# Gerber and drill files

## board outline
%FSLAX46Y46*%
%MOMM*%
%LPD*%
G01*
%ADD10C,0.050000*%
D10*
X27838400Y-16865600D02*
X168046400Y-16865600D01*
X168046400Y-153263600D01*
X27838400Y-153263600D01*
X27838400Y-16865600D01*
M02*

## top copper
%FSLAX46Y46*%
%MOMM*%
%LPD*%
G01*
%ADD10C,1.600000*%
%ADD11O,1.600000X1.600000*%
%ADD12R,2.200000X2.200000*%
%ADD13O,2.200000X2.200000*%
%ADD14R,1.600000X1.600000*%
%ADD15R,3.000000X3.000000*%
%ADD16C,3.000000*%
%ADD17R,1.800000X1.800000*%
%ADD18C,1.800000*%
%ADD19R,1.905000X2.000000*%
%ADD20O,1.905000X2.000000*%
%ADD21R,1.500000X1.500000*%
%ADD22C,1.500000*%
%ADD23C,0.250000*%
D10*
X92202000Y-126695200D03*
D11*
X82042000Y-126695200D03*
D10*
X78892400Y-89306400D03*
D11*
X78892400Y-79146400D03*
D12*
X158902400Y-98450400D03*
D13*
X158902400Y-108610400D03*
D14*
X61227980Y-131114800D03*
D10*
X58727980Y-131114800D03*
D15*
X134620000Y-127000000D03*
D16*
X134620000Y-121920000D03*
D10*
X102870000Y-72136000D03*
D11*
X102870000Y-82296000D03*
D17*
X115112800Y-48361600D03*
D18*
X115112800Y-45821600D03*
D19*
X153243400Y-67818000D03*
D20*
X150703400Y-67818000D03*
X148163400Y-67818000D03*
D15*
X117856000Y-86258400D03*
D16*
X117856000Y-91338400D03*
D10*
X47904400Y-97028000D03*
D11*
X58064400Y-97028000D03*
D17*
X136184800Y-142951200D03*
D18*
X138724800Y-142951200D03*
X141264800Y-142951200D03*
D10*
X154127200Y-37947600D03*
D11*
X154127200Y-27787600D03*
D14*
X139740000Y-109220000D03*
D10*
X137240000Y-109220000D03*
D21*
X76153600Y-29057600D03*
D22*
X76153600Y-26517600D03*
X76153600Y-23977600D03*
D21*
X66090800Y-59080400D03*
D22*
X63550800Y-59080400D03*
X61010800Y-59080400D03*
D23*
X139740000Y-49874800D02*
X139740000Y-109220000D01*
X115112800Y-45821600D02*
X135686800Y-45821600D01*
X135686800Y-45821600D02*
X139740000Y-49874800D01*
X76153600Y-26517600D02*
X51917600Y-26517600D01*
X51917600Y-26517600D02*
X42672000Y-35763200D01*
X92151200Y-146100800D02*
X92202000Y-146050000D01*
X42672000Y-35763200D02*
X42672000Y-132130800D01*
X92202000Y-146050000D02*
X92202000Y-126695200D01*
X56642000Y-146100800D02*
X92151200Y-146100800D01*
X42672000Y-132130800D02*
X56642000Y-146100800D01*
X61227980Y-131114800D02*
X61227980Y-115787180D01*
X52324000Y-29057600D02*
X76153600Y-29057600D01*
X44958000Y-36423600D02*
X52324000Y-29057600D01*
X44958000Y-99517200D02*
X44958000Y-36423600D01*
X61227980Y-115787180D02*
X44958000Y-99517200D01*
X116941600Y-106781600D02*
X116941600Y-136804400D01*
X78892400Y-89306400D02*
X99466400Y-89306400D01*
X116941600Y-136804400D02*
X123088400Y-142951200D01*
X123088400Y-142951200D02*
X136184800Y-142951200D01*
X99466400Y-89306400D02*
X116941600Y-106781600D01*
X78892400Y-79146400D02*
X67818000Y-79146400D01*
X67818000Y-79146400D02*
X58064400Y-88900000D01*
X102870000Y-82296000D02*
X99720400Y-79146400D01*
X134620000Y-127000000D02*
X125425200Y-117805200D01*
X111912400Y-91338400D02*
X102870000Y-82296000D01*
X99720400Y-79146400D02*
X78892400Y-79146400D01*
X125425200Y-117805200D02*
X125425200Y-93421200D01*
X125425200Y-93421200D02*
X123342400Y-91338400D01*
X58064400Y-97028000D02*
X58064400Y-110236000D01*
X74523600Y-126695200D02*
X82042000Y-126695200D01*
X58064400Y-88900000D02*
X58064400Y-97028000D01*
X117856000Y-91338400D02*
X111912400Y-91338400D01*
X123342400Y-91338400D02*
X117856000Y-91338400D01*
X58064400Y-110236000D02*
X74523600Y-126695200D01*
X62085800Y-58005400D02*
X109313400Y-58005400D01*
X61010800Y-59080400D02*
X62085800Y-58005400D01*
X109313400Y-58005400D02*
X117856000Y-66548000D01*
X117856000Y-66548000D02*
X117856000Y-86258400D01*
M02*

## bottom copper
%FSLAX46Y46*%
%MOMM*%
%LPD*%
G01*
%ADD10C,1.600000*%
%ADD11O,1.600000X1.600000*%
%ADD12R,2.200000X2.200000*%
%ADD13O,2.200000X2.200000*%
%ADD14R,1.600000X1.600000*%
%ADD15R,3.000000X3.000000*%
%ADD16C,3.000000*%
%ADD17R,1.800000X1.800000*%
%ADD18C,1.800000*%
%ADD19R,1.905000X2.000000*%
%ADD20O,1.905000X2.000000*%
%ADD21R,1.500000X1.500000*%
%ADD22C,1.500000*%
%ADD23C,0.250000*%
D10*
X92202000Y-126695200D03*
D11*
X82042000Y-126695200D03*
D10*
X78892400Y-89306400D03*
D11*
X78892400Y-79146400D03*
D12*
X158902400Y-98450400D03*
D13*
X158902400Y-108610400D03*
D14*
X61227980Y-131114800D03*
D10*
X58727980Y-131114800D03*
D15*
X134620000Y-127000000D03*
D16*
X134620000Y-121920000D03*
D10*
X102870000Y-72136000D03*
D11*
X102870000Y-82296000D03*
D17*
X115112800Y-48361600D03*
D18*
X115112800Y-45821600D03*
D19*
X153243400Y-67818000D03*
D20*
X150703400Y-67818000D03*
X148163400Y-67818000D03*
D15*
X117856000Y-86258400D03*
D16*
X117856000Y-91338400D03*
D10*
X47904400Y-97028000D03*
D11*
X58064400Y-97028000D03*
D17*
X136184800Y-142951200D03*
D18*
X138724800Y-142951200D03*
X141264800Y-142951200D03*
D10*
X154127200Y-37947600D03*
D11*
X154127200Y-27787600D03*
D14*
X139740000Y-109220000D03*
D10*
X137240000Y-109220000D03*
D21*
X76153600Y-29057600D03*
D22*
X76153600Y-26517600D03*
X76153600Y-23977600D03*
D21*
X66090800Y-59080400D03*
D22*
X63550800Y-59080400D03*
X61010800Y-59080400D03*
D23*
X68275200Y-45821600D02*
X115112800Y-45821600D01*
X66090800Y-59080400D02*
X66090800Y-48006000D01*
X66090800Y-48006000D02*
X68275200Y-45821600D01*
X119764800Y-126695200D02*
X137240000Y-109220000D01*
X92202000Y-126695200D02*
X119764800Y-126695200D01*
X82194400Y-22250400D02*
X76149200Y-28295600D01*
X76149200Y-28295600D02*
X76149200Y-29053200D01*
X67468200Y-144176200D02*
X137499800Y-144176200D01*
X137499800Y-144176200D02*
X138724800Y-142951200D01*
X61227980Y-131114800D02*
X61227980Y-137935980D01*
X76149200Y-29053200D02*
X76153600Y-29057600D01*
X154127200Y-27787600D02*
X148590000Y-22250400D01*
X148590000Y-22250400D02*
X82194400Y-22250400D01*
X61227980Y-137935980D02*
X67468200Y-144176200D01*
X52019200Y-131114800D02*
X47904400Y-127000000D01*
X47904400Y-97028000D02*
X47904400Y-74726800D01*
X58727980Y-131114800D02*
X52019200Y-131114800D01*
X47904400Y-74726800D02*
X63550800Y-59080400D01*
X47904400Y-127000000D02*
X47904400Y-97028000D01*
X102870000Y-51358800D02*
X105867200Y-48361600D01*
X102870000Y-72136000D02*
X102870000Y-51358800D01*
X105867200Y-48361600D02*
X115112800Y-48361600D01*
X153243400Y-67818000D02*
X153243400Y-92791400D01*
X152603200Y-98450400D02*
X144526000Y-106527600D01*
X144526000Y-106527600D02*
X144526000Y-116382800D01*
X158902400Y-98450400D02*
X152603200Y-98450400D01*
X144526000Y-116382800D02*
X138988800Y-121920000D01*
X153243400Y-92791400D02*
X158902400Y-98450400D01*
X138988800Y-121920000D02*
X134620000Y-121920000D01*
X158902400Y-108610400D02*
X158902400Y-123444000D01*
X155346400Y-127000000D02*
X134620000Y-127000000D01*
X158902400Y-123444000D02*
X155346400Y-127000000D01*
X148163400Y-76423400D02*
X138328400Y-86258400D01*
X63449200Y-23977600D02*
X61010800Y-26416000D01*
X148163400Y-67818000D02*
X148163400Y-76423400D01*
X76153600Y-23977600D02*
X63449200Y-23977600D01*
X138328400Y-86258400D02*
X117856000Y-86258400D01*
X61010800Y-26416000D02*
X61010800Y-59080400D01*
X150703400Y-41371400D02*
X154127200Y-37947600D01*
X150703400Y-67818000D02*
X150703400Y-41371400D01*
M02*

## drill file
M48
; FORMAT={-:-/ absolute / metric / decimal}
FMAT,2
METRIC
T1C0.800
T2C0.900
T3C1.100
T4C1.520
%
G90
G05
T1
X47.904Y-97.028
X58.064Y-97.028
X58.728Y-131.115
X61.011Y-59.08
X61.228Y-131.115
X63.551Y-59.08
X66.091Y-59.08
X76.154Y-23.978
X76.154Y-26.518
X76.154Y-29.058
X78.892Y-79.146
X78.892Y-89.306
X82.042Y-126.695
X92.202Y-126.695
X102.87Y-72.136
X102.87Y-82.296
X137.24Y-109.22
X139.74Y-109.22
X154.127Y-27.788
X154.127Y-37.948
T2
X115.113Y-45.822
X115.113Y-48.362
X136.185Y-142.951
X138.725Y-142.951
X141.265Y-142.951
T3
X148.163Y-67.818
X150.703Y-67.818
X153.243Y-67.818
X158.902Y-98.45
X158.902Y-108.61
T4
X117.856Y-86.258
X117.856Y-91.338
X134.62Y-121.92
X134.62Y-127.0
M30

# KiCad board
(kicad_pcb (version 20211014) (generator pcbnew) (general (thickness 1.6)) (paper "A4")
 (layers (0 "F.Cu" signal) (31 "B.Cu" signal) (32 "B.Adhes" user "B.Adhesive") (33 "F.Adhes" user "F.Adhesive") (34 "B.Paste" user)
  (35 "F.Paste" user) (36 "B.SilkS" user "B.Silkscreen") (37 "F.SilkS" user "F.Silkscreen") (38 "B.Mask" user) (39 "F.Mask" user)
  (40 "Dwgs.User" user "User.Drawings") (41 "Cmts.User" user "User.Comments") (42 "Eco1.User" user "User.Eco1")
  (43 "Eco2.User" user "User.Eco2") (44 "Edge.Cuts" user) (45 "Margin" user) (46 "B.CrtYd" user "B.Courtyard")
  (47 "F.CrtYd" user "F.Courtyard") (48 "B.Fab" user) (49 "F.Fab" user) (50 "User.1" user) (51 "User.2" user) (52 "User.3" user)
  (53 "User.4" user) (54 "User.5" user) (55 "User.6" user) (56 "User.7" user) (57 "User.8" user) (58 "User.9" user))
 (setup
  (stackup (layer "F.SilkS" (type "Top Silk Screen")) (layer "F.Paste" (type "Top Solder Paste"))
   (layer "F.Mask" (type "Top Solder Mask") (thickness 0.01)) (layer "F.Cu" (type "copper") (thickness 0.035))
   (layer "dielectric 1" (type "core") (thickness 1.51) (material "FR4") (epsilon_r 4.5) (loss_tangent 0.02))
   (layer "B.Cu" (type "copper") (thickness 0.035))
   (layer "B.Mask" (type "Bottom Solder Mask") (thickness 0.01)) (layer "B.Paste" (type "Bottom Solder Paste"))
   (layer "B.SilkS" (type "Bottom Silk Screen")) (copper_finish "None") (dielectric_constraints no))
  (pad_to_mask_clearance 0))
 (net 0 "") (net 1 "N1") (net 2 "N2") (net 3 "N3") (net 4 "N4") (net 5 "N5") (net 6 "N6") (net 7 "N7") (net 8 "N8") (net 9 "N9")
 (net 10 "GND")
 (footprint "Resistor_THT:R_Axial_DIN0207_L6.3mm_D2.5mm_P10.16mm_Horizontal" (layer "F.Cu") (at 92.202 126.6952 180)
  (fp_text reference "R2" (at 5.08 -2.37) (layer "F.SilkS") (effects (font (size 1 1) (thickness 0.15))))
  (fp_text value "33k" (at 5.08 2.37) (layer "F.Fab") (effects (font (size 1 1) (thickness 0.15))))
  (pad "1" thru_hole circle (at 0 0 180) (size 1.6 1.6) (drill 0.8) (layers *.Cu *.Mask) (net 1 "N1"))
  (pad "2" thru_hole oval (at 10.16 0 180) (size 1.6 1.6) (drill 0.8) (layers *.Cu *.Mask) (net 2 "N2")))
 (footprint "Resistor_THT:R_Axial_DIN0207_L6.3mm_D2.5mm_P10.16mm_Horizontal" (layer "F.Cu") (at 78.8924 89.3064 90)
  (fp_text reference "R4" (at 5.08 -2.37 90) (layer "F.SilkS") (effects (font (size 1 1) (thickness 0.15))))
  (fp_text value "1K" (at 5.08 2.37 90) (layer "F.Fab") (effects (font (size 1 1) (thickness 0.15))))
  (pad "1" thru_hole circle (at 0 0 90) (size 1.6 1.6) (drill 0.8) (layers *.Cu *.Mask) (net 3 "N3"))
  (pad "2" thru_hole oval (at 10.16 0 90) (size 1.6 1.6) (drill 0.8) (layers *.Cu *.Mask) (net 2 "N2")))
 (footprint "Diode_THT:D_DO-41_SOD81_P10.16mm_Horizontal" (layer "F.Cu") (at 158.9024 98.4504 -90)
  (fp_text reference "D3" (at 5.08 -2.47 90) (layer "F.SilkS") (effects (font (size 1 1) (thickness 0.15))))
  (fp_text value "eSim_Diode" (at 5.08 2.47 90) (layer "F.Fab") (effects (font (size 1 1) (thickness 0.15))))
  (pad "1" thru_hole rect (at 0 0 270) (size 2.2 2.2) (drill 1.1) (layers *.Cu *.Mask) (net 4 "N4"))
  (pad "2" thru_hole oval (at 10.16 0 270) (size 2.2 2.2) (drill 1.1) (layers *.Cu *.Mask) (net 2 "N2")))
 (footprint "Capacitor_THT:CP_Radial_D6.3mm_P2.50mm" (layer "F.Cu") (at 61.22798 131.1148 180)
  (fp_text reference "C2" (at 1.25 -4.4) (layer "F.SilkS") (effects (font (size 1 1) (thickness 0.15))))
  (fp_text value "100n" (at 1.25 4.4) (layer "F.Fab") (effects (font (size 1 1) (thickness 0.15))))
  (pad "1" thru_hole rect (at 0 0 180) (size 1.6 1.6) (drill 0.8) (layers *.Cu *.Mask) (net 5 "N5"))
  (pad "2" thru_hole circle (at 2.5 0 180) (size 1.6 1.6) (drill 0.8) (layers *.Cu *.Mask) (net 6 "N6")))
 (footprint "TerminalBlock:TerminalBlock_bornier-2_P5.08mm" (layer "F.Cu") (at 134.62 127 90)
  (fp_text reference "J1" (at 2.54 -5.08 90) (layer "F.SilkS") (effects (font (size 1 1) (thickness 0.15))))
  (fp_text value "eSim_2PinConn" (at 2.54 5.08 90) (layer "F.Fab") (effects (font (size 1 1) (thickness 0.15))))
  (pad "1" thru_hole rect (at 0 0 90) (size 3 3) (drill 1.52) (layers *.Cu *.Mask) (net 2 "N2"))
  (pad "2" thru_hole circle (at 5.08 0 90) (size 3 3) (drill 1.52) (layers *.Cu *.Mask) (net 4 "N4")))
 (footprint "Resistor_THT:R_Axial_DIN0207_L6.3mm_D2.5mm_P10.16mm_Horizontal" (layer "F.Cu") (at 102.87 72.136 -90)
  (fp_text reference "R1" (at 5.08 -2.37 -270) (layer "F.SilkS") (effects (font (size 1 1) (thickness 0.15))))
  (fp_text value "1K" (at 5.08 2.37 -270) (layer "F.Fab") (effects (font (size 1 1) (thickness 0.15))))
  (pad "1" thru_hole circle (at 0 0 270) (size 1.6 1.6) (drill 0.8) (layers *.Cu *.Mask) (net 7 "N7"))
  (pad "2" thru_hole oval (at 10.16 0 270) (size 1.6 1.6) (drill 0.8) (layers *.Cu *.Mask) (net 2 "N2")))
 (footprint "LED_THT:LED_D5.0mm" (layer "F.Cu") (at 115.1128 48.3616 90)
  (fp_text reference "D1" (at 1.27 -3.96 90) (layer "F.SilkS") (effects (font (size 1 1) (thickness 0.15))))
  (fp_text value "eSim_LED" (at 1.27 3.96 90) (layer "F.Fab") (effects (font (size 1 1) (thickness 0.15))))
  (pad "1" thru_hole rect (at 0 0 90) (size 1.8 1.8) (drill 0.9) (layers *.Cu *.Mask) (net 7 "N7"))
  (pad "2" thru_hole circle (at 2.54 0 90) (size 1.8 1.8) (drill 0.9) (layers *.Cu *.Mask) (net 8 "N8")))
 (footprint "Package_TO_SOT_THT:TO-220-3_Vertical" (layer "F.Cu") (at 153.2434 67.818 180)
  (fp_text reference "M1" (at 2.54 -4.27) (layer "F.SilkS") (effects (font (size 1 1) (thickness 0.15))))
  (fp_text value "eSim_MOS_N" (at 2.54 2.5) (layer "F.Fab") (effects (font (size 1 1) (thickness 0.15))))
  (pad "1" thru_hole rect (at 0 0 180) (size 1.905 2) (drill 1.1) (layers *.Cu *.Mask) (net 4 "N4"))
  (pad "2" thru_hole oval (at 2.54 0 180) (size 1.905 2) (drill 1.1) (layers *.Cu *.Mask) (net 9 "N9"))
  (pad "3" thru_hole oval (at 5.08 0 180) (size 1.905 2) (drill 1.1) (layers *.Cu *.Mask) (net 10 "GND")))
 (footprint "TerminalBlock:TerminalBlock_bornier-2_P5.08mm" (layer "F.Cu") (at 117.856 86.2584 -90)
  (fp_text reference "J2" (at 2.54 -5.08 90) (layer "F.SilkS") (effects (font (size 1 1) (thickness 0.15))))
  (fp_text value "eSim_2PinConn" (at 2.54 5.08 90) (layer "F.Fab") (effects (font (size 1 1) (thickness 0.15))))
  (pad "1" thru_hole rect (at 0 0 270) (size 3 3) (drill 1.52) (layers *.Cu *.Mask) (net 10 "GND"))
  (pad "2" thru_hole circle (at 5.08 0 270) (size 3 3) (drill 1.52) (layers *.Cu *.Mask) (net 2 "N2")))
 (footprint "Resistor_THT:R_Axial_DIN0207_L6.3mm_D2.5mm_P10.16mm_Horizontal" (layer "F.Cu") (at 47.9044 97.028)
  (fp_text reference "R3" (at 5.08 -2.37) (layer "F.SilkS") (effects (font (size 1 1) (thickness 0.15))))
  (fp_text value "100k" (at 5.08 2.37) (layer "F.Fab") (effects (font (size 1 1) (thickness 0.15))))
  (pad "1" thru_hole circle (at 0 0) (size 1.6 1.6) (drill 0.8) (layers *.Cu *.Mask) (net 6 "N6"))
  (pad "2" thru_hole oval (at 10.16 0) (size 1.6 1.6) (drill 0.8) (layers *.Cu *.Mask) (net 2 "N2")))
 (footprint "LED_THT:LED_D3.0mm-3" (layer "F.Cu") (at 136.1848 142.9512)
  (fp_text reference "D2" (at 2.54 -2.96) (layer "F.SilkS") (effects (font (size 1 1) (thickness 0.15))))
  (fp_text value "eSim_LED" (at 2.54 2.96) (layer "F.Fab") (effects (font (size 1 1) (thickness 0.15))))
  (pad "1" thru_hole rect (at 0 0) (size 1.8 1.8) (drill 0.9) (layers *.Cu *.Mask) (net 3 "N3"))
  (pad "2" thru_hole circle (at 2.54 0) (size 1.8 1.8) (drill 0.9) (layers *.Cu *.Mask) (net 5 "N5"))
  (pad "3" thru_hole circle (at 5.08 0) (size 1.8 1.8) (drill 0.9) (layers *.Cu *.Mask)))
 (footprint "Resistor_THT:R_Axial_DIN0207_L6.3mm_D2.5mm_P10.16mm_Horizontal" (layer "F.Cu") (at 154.1272 37.9476 90)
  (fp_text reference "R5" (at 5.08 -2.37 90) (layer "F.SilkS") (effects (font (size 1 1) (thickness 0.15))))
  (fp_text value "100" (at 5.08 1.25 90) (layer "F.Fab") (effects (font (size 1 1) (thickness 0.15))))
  (pad "1" thru_hole circle (at 0 0 90) (size 1.6 1.6) (drill 0.8) (layers *.Cu *.Mask) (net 9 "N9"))
  (pad "2" thru_hole oval (at 10.16 0 90) (size 1.6 1.6) (drill 0.8) (layers *.Cu *.Mask) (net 5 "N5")))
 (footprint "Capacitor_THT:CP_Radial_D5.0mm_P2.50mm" (layer "F.Cu") (at 139.74 109.22 180)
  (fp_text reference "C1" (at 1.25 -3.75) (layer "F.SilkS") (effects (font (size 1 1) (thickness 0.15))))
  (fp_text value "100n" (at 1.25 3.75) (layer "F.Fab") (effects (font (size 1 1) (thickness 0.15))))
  (pad "1" thru_hole rect (at 0 0 180) (size 1.6 1.6) (drill 0.8) (layers *.Cu *.Mask) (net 8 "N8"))
  (pad "2" thru_hole circle (at 2.5 0 180) (size 1.6 1.6) (drill 0.8) (layers *.Cu *.Mask) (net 1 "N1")))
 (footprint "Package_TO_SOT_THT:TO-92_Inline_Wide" (layer "F.Cu") (at 76.1536 29.0576 90)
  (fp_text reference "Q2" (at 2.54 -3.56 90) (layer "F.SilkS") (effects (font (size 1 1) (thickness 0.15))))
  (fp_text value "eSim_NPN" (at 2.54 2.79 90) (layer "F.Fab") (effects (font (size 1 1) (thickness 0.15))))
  (pad "1" thru_hole rect (at 0 0 90) (size 1.5 1.5) (drill 0.8) (layers *.Cu *.Mask) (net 5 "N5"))
  (pad "2" thru_hole circle (at 2.54 0 90) (size 1.5 1.5) (drill 0.8) (layers *.Cu *.Mask) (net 1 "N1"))
  (pad "3" thru_hole circle (at 5.08 0 90) (size 1.5 1.5) (drill 0.8) (layers *.Cu *.Mask) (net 10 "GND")))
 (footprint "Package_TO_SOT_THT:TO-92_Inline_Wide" (layer "F.Cu") (at 66.0908 59.0804 180)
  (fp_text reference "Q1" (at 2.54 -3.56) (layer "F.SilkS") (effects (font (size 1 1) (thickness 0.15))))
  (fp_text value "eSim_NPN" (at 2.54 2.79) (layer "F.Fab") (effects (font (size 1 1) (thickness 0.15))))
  (pad "1" thru_hole rect (at 0 0 180) (size 1.5 1.5) (drill 0.8) (layers *.Cu *.Mask) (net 8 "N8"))
  (pad "2" thru_hole circle (at 2.54 0 180) (size 1.5 1.5) (drill 0.8) (layers *.Cu *.Mask) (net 6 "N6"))
  (pad "3" thru_hole circle (at 5.08 0 180) (size 1.5 1.5) (drill 0.8) (layers *.Cu *.Mask) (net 10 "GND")))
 (gr_rect (start 27.8384 16.8656) (end 168.0464 153.2636) (layer "Edge.Cuts") (width 0.05) (fill none))
 (segment (start 139.74 49.8748) (end 139.74 109.22) (width 0.25) (layer "F.Cu") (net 8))
 (segment (start 115.1128 45.8216) (end 135.6868 45.8216) (width 0.25) (layer "F.Cu") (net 8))
 (segment (start 135.6868 45.8216) (end 139.74 49.8748) (width 0.25) (layer "F.Cu") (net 8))
 (segment (start 68.2752 45.8216) (end 115.1128 45.8216) (width 0.25) (layer "B.Cu") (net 8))
 (segment (start 66.0908 59.0804) (end 66.0908 48.006) (width 0.25) (layer "B.Cu") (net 8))
 (segment (start 66.0908 48.006) (end 68.2752 45.8216) (width 0.25) (layer "B.Cu") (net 8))
 (segment (start 76.1536 26.5176) (end 51.9176 26.5176) (width 0.25) (layer "F.Cu") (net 1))
 (segment (start 51.9176 26.5176) (end 42.672 35.7632) (width 0.25) (layer "F.Cu") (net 1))
 (segment (start 92.1512 146.1008) (end 92.202 146.05) (width 0.25) (layer "F.Cu") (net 1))
 (segment (start 42.672 35.7632) (end 42.672 132.1308) (width 0.25) (layer "F.Cu") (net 1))
 (segment (start 92.202 146.05) (end 92.202 126.6952) (width 0.25) (layer "F.Cu") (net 1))
 (segment (start 56.642 146.1008) (end 92.1512 146.1008) (width 0.25) (layer "F.Cu") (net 1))
 (segment (start 42.672 132.1308) (end 56.642 146.1008) (width 0.25) (layer "F.Cu") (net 1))
 (segment (start 119.7648 126.6952) (end 137.24 109.22) (width 0.25) (layer "B.Cu") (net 1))
 (segment (start 92.202 126.6952) (end 119.7648 126.6952) (width 0.25) (layer "B.Cu") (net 1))
 (segment (start 61.22798 131.1148) (end 61.22798 115.78718) (width 0.25) (layer "F.Cu") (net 5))
 (segment (start 52.324 29.0576) (end 76.1536 29.0576) (width 0.25) (layer "F.Cu") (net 5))
 (segment (start 44.958 36.4236) (end 52.324 29.0576) (width 0.25) (layer "F.Cu") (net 5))
 (segment (start 44.958 99.5172) (end 44.958 36.4236) (width 0.25) (layer "F.Cu") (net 5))
 (segment (start 61.22798 115.78718) (end 44.958 99.5172) (width 0.25) (layer "F.Cu") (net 5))
 (segment (start 82.1944 22.2504) (end 76.1492 28.2956) (width 0.25) (layer "B.Cu") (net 5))
 (segment (start 76.1492 28.2956) (end 76.1492 29.0532) (width 0.25) (layer "B.Cu") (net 5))
 (segment (start 67.4682 144.1762) (end 137.4998 144.1762) (width 0.25) (layer "B.Cu") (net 5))
 (segment (start 137.4998 144.1762) (end 138.7248 142.9512) (width 0.25) (layer "B.Cu") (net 5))
 (segment (start 61.22798 131.1148) (end 61.22798 137.93598) (width 0.25) (layer "B.Cu") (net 5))
 (segment (start 76.1492 29.0532) (end 76.1536 29.0576) (width 0.25) (layer "B.Cu") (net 5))
 (segment (start 154.1272 27.7876) (end 148.59 22.2504) (width 0.25) (layer "B.Cu") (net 5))
 (segment (start 148.59 22.2504) (end 82.1944 22.2504) (width 0.25) (layer "B.Cu") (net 5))
 (segment (start 61.22798 137.93598) (end 67.4682 144.1762) (width 0.25) (layer "B.Cu") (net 5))
 (segment (start 52.0192 131.1148) (end 47.9044 127) (width 0.25) (layer "B.Cu") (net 6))
 (segment (start 47.9044 97.028) (end 47.9044 74.7268) (width 0.25) (layer "B.Cu") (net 6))
 (segment (start 58.72798 131.1148) (end 52.0192 131.1148) (width 0.25) (layer "B.Cu") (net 6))
 (segment (start 47.9044 74.7268) (end 63.5508 59.0804) (width 0.25) (layer "B.Cu") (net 6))
 (segment (start 47.9044 127) (end 47.9044 97.028) (width 0.25) (layer "B.Cu") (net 6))
 (segment (start 102.87 51.3588) (end 105.8672 48.3616) (width 0.25) (layer "B.Cu") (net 7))
 (segment (start 102.87 72.136) (end 102.87 51.3588) (width 0.25) (layer "B.Cu") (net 7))
 (segment (start 105.8672 48.3616) (end 115.1128 48.3616) (width 0.25) (layer "B.Cu") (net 7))
 (segment (start 116.9416 106.7816) (end 116.9416 136.8044) (width 0.25) (layer "F.Cu") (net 3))
 (segment (start 78.8924 89.3064) (end 99.4664 89.3064) (width 0.25) (layer "F.Cu") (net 3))
 (segment (start 116.9416 136.8044) (end 123.0884 142.9512) (width 0.25) (layer "F.Cu") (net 3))
 (segment (start 123.0884 142.9512) (end 136.1848 142.9512) (width 0.25) (layer "F.Cu") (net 3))
 (segment (start 99.4664 89.3064) (end 116.9416 106.7816) (width 0.25) (layer "F.Cu") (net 3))
 (segment (start 153.2434 67.818) (end 153.2434 92.7914) (width 0.25) (layer "B.Cu") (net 4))
 (segment (start 152.6032 98.4504) (end 144.526 106.5276) (width 0.25) (layer "B.Cu") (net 4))
 (segment (start 144.526 106.5276) (end 144.526 116.3828) (width 0.25) (layer "B.Cu") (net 4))
 (segment (start 158.9024 98.4504) (end 152.6032 98.4504) (width 0.25) (layer "B.Cu") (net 4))
 (segment (start 144.526 116.3828) (end 138.9888 121.92) (width 0.25) (layer "B.Cu") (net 4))
 (segment (start 153.2434 92.7914) (end 158.9024 98.4504) (width 0.25) (layer "B.Cu") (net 4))
 (segment (start 138.9888 121.92) (end 134.62 121.92) (width 0.25) (layer "B.Cu") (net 4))
 (segment (start 78.8924 79.1464) (end 67.818 79.1464) (width 0.25) (layer "F.Cu") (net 2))
 (segment (start 67.818 79.1464) (end 58.0644 88.9) (width 0.25) (layer "F.Cu") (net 2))
 (segment (start 102.87 82.296) (end 99.7204 79.1464) (width 0.25) (layer "F.Cu") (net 2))
 (segment (start 134.62 127) (end 125.4252 117.8052) (width 0.25) (layer "F.Cu") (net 2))
 (segment (start 111.9124 91.3384) (end 102.87 82.296) (width 0.25) (layer "F.Cu") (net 2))
 (segment (start 99.7204 79.1464) (end 78.8924 79.1464) (width 0.25) (layer "F.Cu") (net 2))
 (segment (start 125.4252 117.8052) (end 125.4252 93.4212) (width 0.25) (layer "F.Cu") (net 2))
 (segment (start 125.4252 93.4212) (end 123.3424 91.3384) (width 0.25) (layer "F.Cu") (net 2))
 (segment (start 58.0644 97.028) (end 58.0644 110.236) (width 0.25) (layer "F.Cu") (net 2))
 (segment (start 74.5236 126.6952) (end 82.042 126.6952) (width 0.25) (layer "F.Cu") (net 2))
 (segment (start 58.0644 88.9) (end 58.0644 97.028) (width 0.25) (layer "F.Cu") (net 2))
 (segment (start 117.856 91.3384) (end 111.9124 91.3384) (width 0.25) (layer "F.Cu") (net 2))
 (segment (start 123.3424 91.3384) (end 117.856 91.3384) (width 0.25) (layer "F.Cu") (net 2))
 (segment (start 58.0644 110.236) (end 74.5236 126.6952) (width 0.25) (layer "F.Cu") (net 2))
 (segment (start 158.9024 108.6104) (end 158.9024 123.444) (width 0.25) (layer "B.Cu") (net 2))
 (segment (start 155.3464 127) (end 134.62 127) (width 0.25) (layer "B.Cu") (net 2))
 (segment (start 158.9024 123.444) (end 155.3464 127) (width 0.25) (layer "B.Cu") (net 2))
 (segment (start 62.0858 58.0054) (end 109.3134 58.0054) (width 0.25) (layer "F.Cu") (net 10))
 (segment (start 61.0108 59.0804) (end 62.0858 58.0054) (width 0.25) (layer "F.Cu") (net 10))
 (segment (start 109.3134 58.0054) (end 117.856 66.548) (width 0.25) (layer "F.Cu") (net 10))
 (segment (start 117.856 66.548) (end 117.856 86.2584) (width 0.25) (layer "F.Cu") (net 10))
 (segment (start 148.1634 76.4234) (end 138.3284 86.2584) (width 0.25) (layer "B.Cu") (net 10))
 (segment (start 63.4492 23.9776) (end 61.0108 26.416) (width 0.25) (layer "B.Cu") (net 10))
 (segment (start 148.1634 67.818) (end 148.1634 76.4234) (width 0.25) (layer "B.Cu") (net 10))
 (segment (start 76.1536 23.9776) (end 63.4492 23.9776) (width 0.25) (layer "B.Cu") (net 10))
 (segment (start 138.3284 86.2584) (end 117.856 86.2584) (width 0.25) (layer "B.Cu") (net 10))
 (segment (start 61.0108 26.416) (end 61.0108 59.0804) (width 0.25) (layer "B.Cu") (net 10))
 (segment (start 150.7034 41.3714) (end 154.1272 37.9476) (width 0.25) (layer "B.Cu") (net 9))
 (segment (start 150.7034 67.818) (end 150.7034 41.3714) (width 0.25) (layer "B.Cu") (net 9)))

